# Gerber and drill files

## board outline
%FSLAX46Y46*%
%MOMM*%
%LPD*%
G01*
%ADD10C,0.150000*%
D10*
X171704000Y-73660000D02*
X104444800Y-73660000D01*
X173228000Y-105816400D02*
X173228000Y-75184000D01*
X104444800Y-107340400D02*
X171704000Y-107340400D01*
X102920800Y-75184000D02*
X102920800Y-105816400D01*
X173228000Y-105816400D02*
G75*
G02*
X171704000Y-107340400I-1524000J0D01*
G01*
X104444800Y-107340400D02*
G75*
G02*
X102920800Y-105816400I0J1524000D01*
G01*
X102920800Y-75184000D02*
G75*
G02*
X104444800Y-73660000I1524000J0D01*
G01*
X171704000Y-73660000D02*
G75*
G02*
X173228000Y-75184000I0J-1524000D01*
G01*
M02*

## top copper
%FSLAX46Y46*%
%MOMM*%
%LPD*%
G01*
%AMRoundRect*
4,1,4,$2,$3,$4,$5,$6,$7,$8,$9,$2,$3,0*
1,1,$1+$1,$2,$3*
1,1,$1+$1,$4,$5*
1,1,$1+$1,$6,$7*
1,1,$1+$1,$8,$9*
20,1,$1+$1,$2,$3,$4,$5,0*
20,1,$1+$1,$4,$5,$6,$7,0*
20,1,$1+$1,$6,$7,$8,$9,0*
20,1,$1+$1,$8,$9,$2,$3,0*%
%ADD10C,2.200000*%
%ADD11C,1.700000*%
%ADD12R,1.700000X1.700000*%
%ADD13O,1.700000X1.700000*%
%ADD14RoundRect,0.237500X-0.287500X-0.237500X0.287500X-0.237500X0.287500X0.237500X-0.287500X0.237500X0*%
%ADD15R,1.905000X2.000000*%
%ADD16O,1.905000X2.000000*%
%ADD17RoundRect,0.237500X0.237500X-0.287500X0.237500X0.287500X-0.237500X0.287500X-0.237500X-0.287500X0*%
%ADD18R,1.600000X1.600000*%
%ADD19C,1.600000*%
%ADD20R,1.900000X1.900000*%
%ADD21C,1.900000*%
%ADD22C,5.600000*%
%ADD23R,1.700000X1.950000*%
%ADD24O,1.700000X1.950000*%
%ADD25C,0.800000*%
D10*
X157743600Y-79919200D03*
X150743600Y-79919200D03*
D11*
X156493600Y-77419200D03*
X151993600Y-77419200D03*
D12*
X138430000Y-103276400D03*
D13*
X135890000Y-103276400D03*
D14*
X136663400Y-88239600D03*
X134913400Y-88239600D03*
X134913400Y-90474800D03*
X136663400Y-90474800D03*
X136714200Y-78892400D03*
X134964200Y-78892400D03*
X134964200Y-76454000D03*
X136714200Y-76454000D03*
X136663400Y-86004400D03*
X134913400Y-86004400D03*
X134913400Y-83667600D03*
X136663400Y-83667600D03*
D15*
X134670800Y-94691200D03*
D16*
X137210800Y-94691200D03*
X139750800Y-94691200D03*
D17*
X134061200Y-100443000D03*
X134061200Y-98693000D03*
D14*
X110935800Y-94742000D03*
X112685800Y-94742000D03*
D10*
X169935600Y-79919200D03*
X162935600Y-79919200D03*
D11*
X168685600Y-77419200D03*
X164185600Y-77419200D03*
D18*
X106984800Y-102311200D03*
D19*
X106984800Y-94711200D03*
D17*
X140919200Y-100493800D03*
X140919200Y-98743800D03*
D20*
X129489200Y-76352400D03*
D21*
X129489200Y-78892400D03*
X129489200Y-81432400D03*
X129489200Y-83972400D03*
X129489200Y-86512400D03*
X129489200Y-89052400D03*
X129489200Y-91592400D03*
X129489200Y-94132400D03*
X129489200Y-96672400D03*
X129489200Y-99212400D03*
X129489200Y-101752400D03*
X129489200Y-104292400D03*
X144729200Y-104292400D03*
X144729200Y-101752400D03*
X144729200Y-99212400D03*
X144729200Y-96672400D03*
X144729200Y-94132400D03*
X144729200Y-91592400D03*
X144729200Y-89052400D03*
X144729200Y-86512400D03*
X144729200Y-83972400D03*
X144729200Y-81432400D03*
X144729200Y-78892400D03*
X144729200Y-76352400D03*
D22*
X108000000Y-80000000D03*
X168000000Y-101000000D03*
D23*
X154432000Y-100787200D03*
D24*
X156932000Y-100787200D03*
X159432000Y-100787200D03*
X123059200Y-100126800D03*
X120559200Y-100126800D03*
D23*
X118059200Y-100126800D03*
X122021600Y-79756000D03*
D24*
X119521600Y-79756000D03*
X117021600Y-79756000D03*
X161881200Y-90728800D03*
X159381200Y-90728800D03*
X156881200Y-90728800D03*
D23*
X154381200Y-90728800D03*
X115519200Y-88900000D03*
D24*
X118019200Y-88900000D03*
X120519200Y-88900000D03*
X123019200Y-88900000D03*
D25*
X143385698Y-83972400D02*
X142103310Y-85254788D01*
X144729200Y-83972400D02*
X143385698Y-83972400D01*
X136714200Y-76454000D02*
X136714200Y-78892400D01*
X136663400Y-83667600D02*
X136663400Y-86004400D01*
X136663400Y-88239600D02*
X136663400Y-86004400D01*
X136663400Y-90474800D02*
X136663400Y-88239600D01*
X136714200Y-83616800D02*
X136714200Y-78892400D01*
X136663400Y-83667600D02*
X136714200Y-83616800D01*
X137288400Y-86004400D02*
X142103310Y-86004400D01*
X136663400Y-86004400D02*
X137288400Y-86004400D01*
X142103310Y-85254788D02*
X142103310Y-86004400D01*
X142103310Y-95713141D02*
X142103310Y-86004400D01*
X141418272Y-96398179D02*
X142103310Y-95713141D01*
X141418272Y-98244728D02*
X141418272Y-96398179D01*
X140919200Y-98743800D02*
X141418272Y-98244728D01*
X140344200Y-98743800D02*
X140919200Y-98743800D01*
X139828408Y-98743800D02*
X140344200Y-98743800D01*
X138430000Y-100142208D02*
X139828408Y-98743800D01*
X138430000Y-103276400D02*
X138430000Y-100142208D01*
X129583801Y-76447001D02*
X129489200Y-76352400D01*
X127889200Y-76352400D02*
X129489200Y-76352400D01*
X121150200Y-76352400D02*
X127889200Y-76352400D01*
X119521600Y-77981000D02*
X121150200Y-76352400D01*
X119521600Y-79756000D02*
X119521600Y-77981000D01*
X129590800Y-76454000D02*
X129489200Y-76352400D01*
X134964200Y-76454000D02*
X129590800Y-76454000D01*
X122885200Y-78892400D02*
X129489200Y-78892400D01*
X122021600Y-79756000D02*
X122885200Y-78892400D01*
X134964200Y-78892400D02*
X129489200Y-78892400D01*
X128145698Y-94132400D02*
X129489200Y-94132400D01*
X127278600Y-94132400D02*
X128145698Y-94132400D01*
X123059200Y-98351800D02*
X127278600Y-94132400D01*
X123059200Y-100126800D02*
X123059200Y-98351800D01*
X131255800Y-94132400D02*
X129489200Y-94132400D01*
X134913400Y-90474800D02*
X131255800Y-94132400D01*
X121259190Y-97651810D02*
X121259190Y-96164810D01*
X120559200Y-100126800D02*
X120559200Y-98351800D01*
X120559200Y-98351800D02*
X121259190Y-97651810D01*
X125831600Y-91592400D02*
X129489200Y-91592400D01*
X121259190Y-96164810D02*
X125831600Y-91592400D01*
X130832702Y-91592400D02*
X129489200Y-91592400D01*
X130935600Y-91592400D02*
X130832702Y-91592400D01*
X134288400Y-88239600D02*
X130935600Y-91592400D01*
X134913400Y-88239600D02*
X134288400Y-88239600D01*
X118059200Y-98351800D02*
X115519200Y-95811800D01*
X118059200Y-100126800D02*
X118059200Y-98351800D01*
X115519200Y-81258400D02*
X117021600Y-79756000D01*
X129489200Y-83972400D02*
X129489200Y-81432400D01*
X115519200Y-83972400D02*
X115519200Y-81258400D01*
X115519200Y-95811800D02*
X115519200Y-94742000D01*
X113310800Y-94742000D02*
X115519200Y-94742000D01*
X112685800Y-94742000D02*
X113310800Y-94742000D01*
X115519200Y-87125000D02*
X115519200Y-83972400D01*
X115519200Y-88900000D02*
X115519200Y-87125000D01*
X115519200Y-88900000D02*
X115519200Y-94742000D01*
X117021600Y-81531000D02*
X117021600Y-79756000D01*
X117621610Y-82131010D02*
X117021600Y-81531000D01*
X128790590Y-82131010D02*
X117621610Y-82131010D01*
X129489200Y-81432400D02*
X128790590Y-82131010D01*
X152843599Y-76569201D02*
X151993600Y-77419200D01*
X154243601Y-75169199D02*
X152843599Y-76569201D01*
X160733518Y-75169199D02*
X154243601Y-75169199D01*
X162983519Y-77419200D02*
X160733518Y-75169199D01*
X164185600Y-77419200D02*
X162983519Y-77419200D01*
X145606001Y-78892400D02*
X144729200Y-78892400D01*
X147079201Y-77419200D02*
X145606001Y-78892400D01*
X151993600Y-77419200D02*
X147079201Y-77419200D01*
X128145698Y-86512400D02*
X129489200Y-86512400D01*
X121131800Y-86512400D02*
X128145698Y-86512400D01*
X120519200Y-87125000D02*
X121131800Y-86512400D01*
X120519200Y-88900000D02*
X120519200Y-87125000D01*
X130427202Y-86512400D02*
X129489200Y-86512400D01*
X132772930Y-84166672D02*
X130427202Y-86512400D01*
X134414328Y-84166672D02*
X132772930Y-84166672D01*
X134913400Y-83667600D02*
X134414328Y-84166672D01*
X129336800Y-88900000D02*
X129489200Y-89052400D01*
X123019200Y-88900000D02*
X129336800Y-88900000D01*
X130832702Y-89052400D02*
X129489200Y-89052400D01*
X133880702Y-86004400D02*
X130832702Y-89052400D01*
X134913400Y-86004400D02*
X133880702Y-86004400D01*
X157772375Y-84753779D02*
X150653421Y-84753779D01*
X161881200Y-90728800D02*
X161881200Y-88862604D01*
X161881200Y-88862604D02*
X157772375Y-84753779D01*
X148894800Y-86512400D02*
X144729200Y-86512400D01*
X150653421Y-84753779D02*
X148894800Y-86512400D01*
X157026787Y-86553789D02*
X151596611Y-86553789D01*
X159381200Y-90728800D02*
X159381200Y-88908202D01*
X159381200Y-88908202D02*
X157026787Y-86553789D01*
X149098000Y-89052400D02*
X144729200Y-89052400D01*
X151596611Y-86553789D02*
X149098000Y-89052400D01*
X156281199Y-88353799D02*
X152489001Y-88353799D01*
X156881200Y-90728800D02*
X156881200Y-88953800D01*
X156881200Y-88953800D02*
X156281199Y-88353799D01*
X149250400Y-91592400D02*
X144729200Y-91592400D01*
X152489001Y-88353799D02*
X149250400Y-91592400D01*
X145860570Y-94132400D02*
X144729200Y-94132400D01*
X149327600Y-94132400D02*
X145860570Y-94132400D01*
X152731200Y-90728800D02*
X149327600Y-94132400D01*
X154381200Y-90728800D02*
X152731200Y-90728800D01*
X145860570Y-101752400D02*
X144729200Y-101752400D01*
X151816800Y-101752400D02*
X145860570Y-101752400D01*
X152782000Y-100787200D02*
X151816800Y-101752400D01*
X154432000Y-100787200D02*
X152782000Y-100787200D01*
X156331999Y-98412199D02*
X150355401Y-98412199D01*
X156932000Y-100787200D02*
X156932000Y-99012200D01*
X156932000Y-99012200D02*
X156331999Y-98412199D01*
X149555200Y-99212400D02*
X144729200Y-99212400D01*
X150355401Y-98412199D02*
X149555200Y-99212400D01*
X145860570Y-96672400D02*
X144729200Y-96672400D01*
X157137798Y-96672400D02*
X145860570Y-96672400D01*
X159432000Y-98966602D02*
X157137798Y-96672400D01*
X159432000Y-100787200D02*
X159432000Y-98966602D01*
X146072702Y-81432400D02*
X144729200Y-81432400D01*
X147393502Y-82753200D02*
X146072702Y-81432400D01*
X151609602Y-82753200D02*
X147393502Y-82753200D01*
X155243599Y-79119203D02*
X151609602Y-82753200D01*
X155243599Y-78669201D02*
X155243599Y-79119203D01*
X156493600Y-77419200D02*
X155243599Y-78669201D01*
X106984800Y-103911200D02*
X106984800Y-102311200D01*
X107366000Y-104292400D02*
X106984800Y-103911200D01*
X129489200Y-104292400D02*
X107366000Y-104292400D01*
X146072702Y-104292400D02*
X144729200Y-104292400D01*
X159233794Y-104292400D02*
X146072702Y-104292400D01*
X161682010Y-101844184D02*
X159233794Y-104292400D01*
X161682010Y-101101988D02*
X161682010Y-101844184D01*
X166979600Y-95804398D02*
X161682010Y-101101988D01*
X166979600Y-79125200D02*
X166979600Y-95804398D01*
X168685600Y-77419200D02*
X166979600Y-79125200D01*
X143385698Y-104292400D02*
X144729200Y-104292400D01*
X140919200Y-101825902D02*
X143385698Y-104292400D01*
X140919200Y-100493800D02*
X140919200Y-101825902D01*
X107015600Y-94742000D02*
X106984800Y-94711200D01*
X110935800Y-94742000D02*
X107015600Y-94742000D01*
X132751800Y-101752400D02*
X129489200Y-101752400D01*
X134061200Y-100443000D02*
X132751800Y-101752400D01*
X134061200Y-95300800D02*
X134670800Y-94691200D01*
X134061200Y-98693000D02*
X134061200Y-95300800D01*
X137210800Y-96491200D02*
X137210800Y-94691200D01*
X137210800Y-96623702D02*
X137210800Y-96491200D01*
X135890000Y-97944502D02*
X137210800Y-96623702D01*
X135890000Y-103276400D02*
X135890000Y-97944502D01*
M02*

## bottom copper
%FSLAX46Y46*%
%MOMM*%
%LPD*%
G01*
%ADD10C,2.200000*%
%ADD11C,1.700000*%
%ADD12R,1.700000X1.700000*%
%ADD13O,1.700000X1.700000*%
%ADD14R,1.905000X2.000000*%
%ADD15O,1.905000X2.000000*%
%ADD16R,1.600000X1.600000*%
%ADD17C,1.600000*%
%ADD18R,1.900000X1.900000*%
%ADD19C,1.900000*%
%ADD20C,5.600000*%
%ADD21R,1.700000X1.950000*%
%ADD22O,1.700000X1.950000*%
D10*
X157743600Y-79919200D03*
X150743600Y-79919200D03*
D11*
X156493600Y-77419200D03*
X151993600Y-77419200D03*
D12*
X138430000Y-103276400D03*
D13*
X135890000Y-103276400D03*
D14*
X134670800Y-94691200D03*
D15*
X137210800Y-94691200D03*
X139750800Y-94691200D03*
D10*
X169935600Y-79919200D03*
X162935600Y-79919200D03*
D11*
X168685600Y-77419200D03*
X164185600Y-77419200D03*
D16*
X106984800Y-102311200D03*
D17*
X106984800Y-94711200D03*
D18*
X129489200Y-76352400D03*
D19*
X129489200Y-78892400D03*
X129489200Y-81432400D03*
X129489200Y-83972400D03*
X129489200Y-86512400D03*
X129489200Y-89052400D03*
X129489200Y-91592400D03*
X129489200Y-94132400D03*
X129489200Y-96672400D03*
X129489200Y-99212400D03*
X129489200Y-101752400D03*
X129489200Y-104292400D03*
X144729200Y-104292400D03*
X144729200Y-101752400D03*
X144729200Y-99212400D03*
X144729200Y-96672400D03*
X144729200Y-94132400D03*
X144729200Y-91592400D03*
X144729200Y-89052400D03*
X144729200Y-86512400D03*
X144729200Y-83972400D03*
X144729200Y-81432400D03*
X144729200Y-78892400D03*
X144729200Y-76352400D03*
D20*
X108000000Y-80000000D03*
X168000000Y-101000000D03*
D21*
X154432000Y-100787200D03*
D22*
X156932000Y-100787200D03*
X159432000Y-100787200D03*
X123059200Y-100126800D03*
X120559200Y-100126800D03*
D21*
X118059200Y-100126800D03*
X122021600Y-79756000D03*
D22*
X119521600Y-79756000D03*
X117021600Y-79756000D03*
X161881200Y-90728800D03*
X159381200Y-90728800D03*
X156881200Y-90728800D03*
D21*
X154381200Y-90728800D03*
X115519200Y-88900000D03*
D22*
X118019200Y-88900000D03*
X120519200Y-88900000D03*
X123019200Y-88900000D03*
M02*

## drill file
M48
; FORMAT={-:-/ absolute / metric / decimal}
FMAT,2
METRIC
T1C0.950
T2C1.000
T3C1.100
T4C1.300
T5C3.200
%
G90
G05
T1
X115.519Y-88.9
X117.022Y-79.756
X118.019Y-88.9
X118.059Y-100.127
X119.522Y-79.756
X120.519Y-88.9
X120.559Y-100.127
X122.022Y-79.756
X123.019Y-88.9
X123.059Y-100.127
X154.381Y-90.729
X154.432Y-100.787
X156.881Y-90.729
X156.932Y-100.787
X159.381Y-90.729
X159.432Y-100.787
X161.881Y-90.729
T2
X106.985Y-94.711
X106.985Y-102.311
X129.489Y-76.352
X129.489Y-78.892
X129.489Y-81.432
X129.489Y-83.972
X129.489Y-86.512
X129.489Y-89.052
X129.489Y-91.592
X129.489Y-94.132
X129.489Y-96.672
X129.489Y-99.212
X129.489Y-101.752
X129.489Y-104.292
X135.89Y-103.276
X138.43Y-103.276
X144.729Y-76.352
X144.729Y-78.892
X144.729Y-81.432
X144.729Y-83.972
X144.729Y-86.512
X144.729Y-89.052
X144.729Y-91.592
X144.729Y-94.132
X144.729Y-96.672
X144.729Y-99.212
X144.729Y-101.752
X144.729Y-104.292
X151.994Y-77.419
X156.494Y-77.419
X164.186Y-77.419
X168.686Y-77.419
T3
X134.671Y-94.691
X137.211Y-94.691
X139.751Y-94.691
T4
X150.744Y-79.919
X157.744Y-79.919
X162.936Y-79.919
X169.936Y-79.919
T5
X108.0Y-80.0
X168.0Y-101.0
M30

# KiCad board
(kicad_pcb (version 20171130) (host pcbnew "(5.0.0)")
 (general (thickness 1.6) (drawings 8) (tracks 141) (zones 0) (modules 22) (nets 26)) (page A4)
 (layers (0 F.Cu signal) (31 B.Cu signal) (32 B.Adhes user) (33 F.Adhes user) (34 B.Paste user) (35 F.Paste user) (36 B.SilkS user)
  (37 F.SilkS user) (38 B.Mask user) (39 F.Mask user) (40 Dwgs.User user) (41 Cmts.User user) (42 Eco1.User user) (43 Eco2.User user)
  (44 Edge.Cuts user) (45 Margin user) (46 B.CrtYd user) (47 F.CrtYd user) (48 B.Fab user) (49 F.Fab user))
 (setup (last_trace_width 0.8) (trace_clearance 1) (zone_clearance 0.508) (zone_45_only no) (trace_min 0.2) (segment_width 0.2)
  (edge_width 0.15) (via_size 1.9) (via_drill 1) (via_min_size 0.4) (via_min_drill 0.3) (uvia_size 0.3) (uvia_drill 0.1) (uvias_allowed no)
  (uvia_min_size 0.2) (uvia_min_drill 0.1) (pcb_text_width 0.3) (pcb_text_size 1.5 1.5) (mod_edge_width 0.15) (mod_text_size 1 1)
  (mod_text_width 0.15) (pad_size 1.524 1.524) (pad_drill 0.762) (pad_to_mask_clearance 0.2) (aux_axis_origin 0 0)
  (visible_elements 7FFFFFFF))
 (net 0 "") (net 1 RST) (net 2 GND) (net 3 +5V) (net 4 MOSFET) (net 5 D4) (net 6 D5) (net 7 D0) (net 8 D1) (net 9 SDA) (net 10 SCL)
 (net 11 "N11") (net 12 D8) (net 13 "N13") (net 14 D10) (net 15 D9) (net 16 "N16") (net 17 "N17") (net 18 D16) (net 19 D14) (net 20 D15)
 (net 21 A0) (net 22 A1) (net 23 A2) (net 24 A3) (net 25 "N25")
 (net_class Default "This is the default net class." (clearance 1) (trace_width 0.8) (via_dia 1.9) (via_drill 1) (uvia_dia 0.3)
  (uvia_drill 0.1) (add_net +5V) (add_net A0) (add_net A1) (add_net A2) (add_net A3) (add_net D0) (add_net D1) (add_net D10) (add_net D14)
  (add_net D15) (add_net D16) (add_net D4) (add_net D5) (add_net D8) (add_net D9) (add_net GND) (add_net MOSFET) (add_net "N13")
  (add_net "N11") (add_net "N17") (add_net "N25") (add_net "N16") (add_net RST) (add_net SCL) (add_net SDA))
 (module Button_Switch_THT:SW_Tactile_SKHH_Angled (layer F.Cu) (at 151.9936 77.4192)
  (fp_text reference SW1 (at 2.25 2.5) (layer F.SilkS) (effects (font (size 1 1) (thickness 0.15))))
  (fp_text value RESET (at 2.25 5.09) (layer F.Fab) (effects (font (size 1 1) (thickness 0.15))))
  (pad "" thru_hole circle (at 5.75 2.5 180) (size 2.2 2.2) (drill 1.3) (layers *.Cu *.Mask))
  (pad "" thru_hole circle (at -1.25 2.5 180) (size 2.2 2.2) (drill 1.3) (layers *.Cu *.Mask))
  (pad 2 thru_hole circle (at 4.5 0 180) (size 1.7 1.7) (drill 1) (layers *.Cu *.Mask) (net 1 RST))
  (pad 1 thru_hole circle (at 0 0 180) (size 1.7 1.7) (drill 1) (layers *.Cu *.Mask) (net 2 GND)))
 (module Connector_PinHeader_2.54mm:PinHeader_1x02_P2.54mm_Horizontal (layer F.Cu) (at 138.43 103.2764 270)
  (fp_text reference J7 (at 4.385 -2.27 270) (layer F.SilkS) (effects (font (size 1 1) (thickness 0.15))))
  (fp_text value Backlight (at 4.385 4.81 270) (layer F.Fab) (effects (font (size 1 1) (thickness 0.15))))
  (pad 1 thru_hole rect (at 0 0 270) (size 1.7 1.7) (drill 1) (layers *.Cu *.Mask) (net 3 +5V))
  (pad 2 thru_hole oval (at 0 2.54 270) (size 1.7 1.7) (drill 1) (layers *.Cu *.Mask) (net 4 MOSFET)))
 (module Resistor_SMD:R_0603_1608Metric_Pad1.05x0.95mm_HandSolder (layer F.Cu) (at 135.7884 88.2396)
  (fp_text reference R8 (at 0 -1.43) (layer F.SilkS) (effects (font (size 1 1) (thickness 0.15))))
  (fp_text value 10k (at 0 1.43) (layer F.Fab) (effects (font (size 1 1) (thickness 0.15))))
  (pad 2 smd roundrect (at 0.875 0) (size 1.05 0.95) (layers F.Cu F.Paste F.Mask) (roundrect_rratio 0.25) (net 3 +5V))
  (pad 1 smd roundrect (at -0.875 0) (size 1.05 0.95) (layers F.Cu F.Paste F.Mask) (roundrect_rratio 0.25) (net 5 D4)))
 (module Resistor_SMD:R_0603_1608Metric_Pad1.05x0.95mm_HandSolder (layer F.Cu) (at 135.7884 90.4748)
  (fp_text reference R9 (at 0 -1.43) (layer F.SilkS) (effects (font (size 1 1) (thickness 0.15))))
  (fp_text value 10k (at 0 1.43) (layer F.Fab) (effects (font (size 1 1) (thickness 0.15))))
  (pad 1 smd roundrect (at -0.875 0) (size 1.05 0.95) (layers F.Cu F.Paste F.Mask) (roundrect_rratio 0.25) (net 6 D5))
  (pad 2 smd roundrect (at 0.875 0) (size 1.05 0.95) (layers F.Cu F.Paste F.Mask) (roundrect_rratio 0.25) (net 3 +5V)))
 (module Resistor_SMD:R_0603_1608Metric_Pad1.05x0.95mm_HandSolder (layer F.Cu) (at 135.8392 78.8924)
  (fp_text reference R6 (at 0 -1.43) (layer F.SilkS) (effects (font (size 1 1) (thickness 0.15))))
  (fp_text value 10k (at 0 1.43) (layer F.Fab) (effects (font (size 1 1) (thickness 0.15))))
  (pad 2 smd roundrect (at 0.875 0) (size 1.05 0.95) (layers F.Cu F.Paste F.Mask) (roundrect_rratio 0.25) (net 3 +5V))
  (pad 1 smd roundrect (at -0.875 0) (size 1.05 0.95) (layers F.Cu F.Paste F.Mask) (roundrect_rratio 0.25) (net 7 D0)))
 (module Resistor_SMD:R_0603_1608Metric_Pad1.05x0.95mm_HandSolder (layer F.Cu) (at 135.8392 76.454)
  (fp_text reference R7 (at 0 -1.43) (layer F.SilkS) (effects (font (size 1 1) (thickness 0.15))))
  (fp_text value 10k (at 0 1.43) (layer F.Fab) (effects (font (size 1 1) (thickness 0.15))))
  (pad 1 smd roundrect (at -0.875 0) (size 1.05 0.95) (layers F.Cu F.Paste F.Mask) (roundrect_rratio 0.25) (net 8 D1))
  (pad 2 smd roundrect (at 0.875 0) (size 1.05 0.95) (layers F.Cu F.Paste F.Mask) (roundrect_rratio 0.25) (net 3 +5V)))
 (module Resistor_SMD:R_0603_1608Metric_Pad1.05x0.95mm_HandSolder (layer F.Cu) (at 135.7884 86.0044)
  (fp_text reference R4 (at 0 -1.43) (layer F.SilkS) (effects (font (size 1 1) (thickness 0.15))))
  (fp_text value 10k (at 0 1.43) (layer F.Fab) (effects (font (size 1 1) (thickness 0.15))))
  (pad 2 smd roundrect (at 0.875 0) (size 1.05 0.95) (layers F.Cu F.Paste F.Mask) (roundrect_rratio 0.25) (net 3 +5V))
  (pad 1 smd roundrect (at -0.875 0) (size 1.05 0.95) (layers F.Cu F.Paste F.Mask) (roundrect_rratio 0.25) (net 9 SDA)))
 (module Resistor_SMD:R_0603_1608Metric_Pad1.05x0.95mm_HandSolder (layer F.Cu) (at 135.7884 83.6676)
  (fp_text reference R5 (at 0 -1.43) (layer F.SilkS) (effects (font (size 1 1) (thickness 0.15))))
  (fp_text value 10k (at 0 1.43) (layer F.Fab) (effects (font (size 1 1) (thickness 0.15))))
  (pad 1 smd roundrect (at -0.875 0) (size 1.05 0.95) (layers F.Cu F.Paste F.Mask) (roundrect_rratio 0.25) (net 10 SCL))
  (pad 2 smd roundrect (at 0.875 0) (size 1.05 0.95) (layers F.Cu F.Paste F.Mask) (roundrect_rratio 0.25) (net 3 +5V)))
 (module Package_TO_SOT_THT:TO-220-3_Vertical (layer F.Cu) (at 134.6708 94.6912)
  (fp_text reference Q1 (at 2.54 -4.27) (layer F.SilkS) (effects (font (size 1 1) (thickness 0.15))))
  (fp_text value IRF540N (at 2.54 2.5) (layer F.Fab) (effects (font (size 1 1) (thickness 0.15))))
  (pad 1 thru_hole rect (at 0 0) (size 1.905 2) (drill 1.1) (layers *.Cu *.Mask) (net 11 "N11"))
  (pad 2 thru_hole oval (at 2.54 0) (size 1.905 2) (drill 1.1) (layers *.Cu *.Mask) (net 4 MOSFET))
  (pad 3 thru_hole oval (at 5.08 0) (size 1.905 2) (drill 1.1) (layers *.Cu *.Mask) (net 2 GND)))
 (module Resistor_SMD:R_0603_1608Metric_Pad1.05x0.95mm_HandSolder (layer F.Cu) (at 134.0612 99.568 90)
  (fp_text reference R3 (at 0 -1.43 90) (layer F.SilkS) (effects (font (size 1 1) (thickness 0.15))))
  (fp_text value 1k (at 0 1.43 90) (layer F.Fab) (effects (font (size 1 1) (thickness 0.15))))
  (pad 1 smd roundrect (at -0.875 0 90) (size 1.05 0.95) (layers F.Cu F.Paste F.Mask) (roundrect_rratio 0.25) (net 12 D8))
  (pad 2 smd roundrect (at 0.875 0 90) (size 1.05 0.95) (layers F.Cu F.Paste F.Mask) (roundrect_rratio 0.25) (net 11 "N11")))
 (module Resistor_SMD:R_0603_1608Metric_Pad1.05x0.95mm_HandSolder (layer F.Cu) (at 111.8108 94.742)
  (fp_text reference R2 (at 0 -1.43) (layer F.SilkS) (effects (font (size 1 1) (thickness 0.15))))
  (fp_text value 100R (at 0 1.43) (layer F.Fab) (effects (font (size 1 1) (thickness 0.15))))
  (pad 1 smd roundrect (at -0.875 0) (size 1.05 0.95) (layers F.Cu F.Paste F.Mask) (roundrect_rratio 0.25) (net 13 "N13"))
  (pad 2 smd roundrect (at 0.875 0) (size 1.05 0.95) (layers F.Cu F.Paste F.Mask) (roundrect_rratio 0.25) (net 2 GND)))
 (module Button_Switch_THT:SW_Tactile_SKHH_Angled (layer F.Cu) (at 164.1856 77.4192)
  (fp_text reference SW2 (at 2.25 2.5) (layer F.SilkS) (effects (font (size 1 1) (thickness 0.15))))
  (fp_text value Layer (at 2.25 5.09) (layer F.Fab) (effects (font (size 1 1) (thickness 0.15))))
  (pad "" thru_hole circle (at 5.75 2.5 180) (size 2.2 2.2) (drill 1.3) (layers *.Cu *.Mask))
  (pad "" thru_hole circle (at -1.25 2.5 180) (size 2.2 2.2) (drill 1.3) (layers *.Cu *.Mask))
  (pad 2 thru_hole circle (at 4.5 0 180) (size 1.7 1.7) (drill 1) (layers *.Cu *.Mask) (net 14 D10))
  (pad 1 thru_hole circle (at 0 0 180) (size 1.7 1.7) (drill 1) (layers *.Cu *.Mask) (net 2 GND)))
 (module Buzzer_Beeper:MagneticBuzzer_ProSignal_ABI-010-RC (layer F.Cu) (at 106.9848 102.3112 90)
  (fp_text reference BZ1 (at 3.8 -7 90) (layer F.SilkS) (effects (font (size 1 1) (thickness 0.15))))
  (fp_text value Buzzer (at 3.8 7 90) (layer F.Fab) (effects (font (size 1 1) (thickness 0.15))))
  (pad 1 thru_hole rect (at 0 0 90) (size 1.6 1.6) (drill 1) (layers *.Cu *.Mask) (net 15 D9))
  (pad 2 thru_hole circle (at 7.6 0 90) (size 1.6 1.6) (drill 1) (layers *.Cu *.Mask) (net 13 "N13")))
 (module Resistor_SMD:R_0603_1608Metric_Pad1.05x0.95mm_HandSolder (layer F.Cu) (at 140.9192 99.6188 90)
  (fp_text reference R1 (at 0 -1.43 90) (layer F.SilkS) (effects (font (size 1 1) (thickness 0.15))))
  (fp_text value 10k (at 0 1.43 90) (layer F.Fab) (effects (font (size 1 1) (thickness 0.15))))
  (pad 1 smd roundrect (at -0.875 0 90) (size 1.05 0.95) (layers F.Cu F.Paste F.Mask) (roundrect_rratio 0.25) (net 14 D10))
  (pad 2 smd roundrect (at 0.875 0 90) (size 1.05 0.95) (layers F.Cu F.Paste F.Mask) (roundrect_rratio 0.25) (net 3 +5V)))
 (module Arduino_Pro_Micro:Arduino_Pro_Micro (layer F.Cu) (at 137.1092 90.3224 270)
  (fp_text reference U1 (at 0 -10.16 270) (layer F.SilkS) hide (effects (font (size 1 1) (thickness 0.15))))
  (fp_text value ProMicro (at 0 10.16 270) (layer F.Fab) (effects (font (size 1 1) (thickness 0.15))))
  (pad 1 thru_hole rect (at -13.97 7.62 270) (size 1.9 1.9) (drill 1) (layers *.Cu *.Mask F.SilkS) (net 8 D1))
  (pad 2 thru_hole circle (at -11.43 7.62 270) (size 1.9 1.9) (drill 1) (layers *.Cu *.Mask F.SilkS) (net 7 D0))
  (pad 3 thru_hole circle (at -8.89 7.62 270) (size 1.9 1.9) (drill 1) (layers *.Cu *.Mask F.SilkS) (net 2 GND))
  (pad 4 thru_hole circle (at -6.35 7.62 270) (size 1.9 1.9) (drill 1) (layers *.Cu *.Mask F.SilkS) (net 2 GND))
  (pad 5 thru_hole circle (at -3.81 7.62 270) (size 1.9 1.9) (drill 1) (layers *.Cu *.Mask F.SilkS) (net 10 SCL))
  (pad 6 thru_hole circle (at -1.27 7.62 270) (size 1.9 1.9) (drill 1) (layers *.Cu *.Mask F.SilkS) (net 9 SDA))
  (pad 7 thru_hole circle (at 1.27 7.62 270) (size 1.9 1.9) (drill 1) (layers *.Cu *.Mask F.SilkS) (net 5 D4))
  (pad 8 thru_hole circle (at 3.81 7.62 270) (size 1.9 1.9) (drill 1) (layers *.Cu *.Mask F.SilkS) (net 6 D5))
  (pad 9 thru_hole circle (at 6.35 7.62 270) (size 1.9 1.9) (drill 1) (layers *.Cu *.Mask F.SilkS) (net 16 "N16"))
  (pad 10 thru_hole circle (at 8.89 7.62 270) (size 1.9 1.9) (drill 1) (layers *.Cu *.Mask F.SilkS) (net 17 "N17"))
  (pad 11 thru_hole circle (at 11.43 7.62 270) (size 1.9 1.9) (drill 1) (layers *.Cu *.Mask F.SilkS) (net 12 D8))
  (pad 12 thru_hole circle (at 13.97 7.62 270) (size 1.9 1.9) (drill 1) (layers *.Cu *.Mask F.SilkS) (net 15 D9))
  (pad 13 thru_hole circle (at 13.97 -7.62 270) (size 1.9 1.9) (drill 1) (layers *.Cu *.Mask F.SilkS) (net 14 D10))
  (pad 14 thru_hole circle (at 11.43 -7.62 270) (size 1.9 1.9) (drill 1) (layers *.Cu *.Mask F.SilkS) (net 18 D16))
  (pad 15 thru_hole circle (at 8.89 -7.62 270) (size 1.9 1.9) (drill 1) (layers *.Cu *.Mask F.SilkS) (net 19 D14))
  (pad 16 thru_hole circle (at 6.35 -7.62 270) (size 1.9 1.9) (drill 1) (layers *.Cu *.Mask F.SilkS) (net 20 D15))
  (pad 17 thru_hole circle (at 3.81 -7.62 270) (size 1.9 1.9) (drill 1) (layers *.Cu *.Mask F.SilkS) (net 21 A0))
  (pad 18 thru_hole circle (at 1.27 -7.62 270) (size 1.9 1.9) (drill 1) (layers *.Cu *.Mask F.SilkS) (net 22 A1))
  (pad 19 thru_hole circle (at -1.27 -7.62 270) (size 1.9 1.9) (drill 1) (layers *.Cu *.Mask F.SilkS) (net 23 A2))
  (pad 20 thru_hole circle (at -3.81 -7.62 270) (size 1.9 1.9) (drill 1) (layers *.Cu *.Mask F.SilkS) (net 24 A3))
  (pad 21 thru_hole circle (at -6.35 -7.62 270) (size 1.9 1.9) (drill 1) (layers *.Cu *.Mask F.SilkS) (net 3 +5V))
  (pad 22 thru_hole circle (at -8.89 -7.62 270) (size 1.9 1.9) (drill 1) (layers *.Cu *.Mask F.SilkS) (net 1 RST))
  (pad 23 thru_hole circle (at -11.43 -7.62 270) (size 1.9 1.9) (drill 1) (layers *.Cu *.Mask F.SilkS) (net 2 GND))
  (pad 24 thru_hole circle (at -13.97 -7.62 270) (size 1.9 1.9) (drill 1) (layers *.Cu *.Mask F.SilkS) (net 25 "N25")))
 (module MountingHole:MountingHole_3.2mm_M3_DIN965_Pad (layer F.Cu) (at 108 80)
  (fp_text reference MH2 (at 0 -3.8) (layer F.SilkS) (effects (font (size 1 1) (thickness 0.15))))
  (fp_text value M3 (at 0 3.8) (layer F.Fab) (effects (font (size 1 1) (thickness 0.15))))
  (pad 1 thru_hole circle (at 0 0) (size 5.6 5.6) (drill 3.2) (layers *.Cu *.Mask)))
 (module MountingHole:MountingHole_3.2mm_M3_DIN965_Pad (layer F.Cu) (at 168 101)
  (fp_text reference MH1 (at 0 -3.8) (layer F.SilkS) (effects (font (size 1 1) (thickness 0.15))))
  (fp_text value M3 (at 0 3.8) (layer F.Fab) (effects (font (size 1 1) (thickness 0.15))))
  (pad 1 thru_hole circle (at 0 0) (size 5.6 5.6) (drill 3.2) (layers *.Cu *.Mask)))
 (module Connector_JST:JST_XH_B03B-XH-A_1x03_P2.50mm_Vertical (layer F.Cu) (at 154.432 100.7872)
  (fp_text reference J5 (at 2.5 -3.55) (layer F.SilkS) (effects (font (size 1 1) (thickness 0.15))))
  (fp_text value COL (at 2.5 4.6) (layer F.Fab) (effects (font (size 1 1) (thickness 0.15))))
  (pad 1 thru_hole rect (at 0 0) (size 1.7 1.95) (drill 0.95) (layers *.Cu *.Mask) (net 18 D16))
  (pad 2 thru_hole oval (at 2.5 0) (size 1.7 1.95) (drill 0.95) (layers *.Cu *.Mask) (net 19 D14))
  (pad 3 thru_hole oval (at 5 0) (size 1.7 1.95) (drill 0.95) (layers *.Cu *.Mask) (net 20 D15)))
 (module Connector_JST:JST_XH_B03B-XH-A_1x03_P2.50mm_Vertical (layer F.Cu) (at 118.0592 100.1268)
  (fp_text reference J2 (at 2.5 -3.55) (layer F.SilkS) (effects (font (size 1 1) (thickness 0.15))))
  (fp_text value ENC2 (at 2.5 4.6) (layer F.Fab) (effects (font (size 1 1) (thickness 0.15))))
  (pad 3 thru_hole oval (at 5 0) (size 1.7 1.95) (drill 0.95) (layers *.Cu *.Mask) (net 6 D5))
  (pad 2 thru_hole oval (at 2.5 0) (size 1.7 1.95) (drill 0.95) (layers *.Cu *.Mask) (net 5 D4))
  (pad 1 thru_hole rect (at 0 0) (size 1.7 1.95) (drill 0.95) (layers *.Cu *.Mask) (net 2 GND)))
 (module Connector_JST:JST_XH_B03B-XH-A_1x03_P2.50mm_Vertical (layer F.Cu) (at 122.0216 79.756 180)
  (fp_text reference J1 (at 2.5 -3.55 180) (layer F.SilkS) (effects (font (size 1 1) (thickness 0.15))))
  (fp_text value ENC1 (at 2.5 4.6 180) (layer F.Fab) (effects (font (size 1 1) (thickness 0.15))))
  (pad 1 thru_hole rect (at 0 0 180) (size 1.7 1.95) (drill 0.95) (layers *.Cu *.Mask) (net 7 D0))
  (pad 2 thru_hole oval (at 2.5 0 180) (size 1.7 1.95) (drill 0.95) (layers *.Cu *.Mask) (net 8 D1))
  (pad 3 thru_hole oval (at 5 0 180) (size 1.7 1.95) (drill 0.95) (layers *.Cu *.Mask) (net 2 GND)))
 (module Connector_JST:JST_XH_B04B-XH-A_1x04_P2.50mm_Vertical (layer F.Cu) (at 154.3812 90.7288)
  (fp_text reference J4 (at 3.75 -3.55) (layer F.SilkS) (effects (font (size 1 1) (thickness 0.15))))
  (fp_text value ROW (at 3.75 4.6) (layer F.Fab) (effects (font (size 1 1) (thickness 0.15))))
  (pad 4 thru_hole oval (at 7.5 0) (size 1.7 1.95) (drill 0.95) (layers *.Cu *.Mask) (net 24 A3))
  (pad 3 thru_hole oval (at 5 0) (size 1.7 1.95) (drill 0.95) (layers *.Cu *.Mask) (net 23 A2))
  (pad 2 thru_hole oval (at 2.5 0) (size 1.7 1.95) (drill 0.95) (layers *.Cu *.Mask) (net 22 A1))
  (pad 1 thru_hole rect (at 0 0) (size 1.7 1.95) (drill 0.95) (layers *.Cu *.Mask) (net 21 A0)))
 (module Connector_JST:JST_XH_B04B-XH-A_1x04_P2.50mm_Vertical (layer F.Cu) (at 115.5192 88.9)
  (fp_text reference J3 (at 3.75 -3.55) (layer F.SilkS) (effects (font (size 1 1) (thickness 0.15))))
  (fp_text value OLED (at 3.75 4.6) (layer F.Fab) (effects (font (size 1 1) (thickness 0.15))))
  (pad 1 thru_hole rect (at 0 0) (size 1.7 1.95) (drill 0.95) (layers *.Cu *.Mask) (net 2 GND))
  (pad 2 thru_hole oval (at 2.5 0) (size 1.7 1.95) (drill 0.95) (layers *.Cu *.Mask) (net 3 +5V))
  (pad 3 thru_hole oval (at 5 0) (size 1.7 1.95) (drill 0.95) (layers *.Cu *.Mask) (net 10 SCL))
  (pad 4 thru_hole oval (at 7.5 0) (size 1.7 1.95) (drill 0.95) (layers *.Cu *.Mask) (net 9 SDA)))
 (gr_line (start 171.704 73.66) (end 104.4448 73.66) (layer Edge.Cuts) (width 0.15))
 (gr_line (start 173.228 105.8164) (end 173.228 75.184) (layer Edge.Cuts) (width 0.15))
 (gr_line (start 104.4448 107.3404) (end 171.704 107.3404) (layer Edge.Cuts) (width 0.15))
 (gr_line (start 102.9208 75.184) (end 102.9208 105.8164) (layer Edge.Cuts) (width 0.15))
 (gr_arc (start 171.704 105.8164) (end 171.704 107.3404) (angle -90) (layer Edge.Cuts) (width 0.15))
 (gr_arc (start 104.4448 105.8164) (end 102.9208 105.8164) (angle -90) (layer Edge.Cuts) (width 0.15))
 (gr_arc (start 104.4448 75.184) (end 104.4448 73.66) (angle -90) (layer Edge.Cuts) (width 0.15))
 (gr_arc (start 171.704 75.184) (end 173.228 75.184) (angle -90) (layer Edge.Cuts) (width 0.15))
 (segment (start 143.385698 83.9724) (end 142.10331 85.254788) (width 0.8) (layer F.Cu) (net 3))
 (segment (start 144.7292 83.9724) (end 143.385698 83.9724) (width 0.8) (layer F.Cu) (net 3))
 (segment (start 136.7142 76.454) (end 136.7142 78.8924) (width 0.8) (layer F.Cu) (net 3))
 (segment (start 136.6634 83.6676) (end 136.6634 86.0044) (width 0.8) (layer F.Cu) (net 3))
 (segment (start 136.6634 88.2396) (end 136.6634 86.0044) (width 0.8) (layer F.Cu) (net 3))
 (segment (start 136.6634 90.4748) (end 136.6634 88.2396) (width 0.8) (layer F.Cu) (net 3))
 (segment (start 136.7142 83.6168) (end 136.7142 78.8924) (width 0.8) (layer F.Cu) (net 3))
 (segment (start 136.6634 83.6676) (end 136.7142 83.6168) (width 0.8) (layer F.Cu) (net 3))
 (segment (start 137.2884 86.0044) (end 142.10331 86.0044) (width 0.8) (layer F.Cu) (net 3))
 (segment (start 136.6634 86.0044) (end 137.2884 86.0044) (width 0.8) (layer F.Cu) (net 3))
 (segment (start 142.10331 85.254788) (end 142.10331 86.0044) (width 0.8) (layer F.Cu) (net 3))
 (segment (start 142.10331 95.713141) (end 142.10331 86.0044) (width 0.8) (layer F.Cu) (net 3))
 (segment (start 141.418272 96.398179) (end 142.10331 95.713141) (width 0.8) (layer F.Cu) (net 3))
 (segment (start 141.418272 98.244728) (end 141.418272 96.398179) (width 0.8) (layer F.Cu) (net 3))
 (segment (start 140.9192 98.7438) (end 141.418272 98.244728) (width 0.8) (layer F.Cu) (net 3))
 (segment (start 140.3442 98.7438) (end 140.9192 98.7438) (width 0.8) (layer F.Cu) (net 3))
 (segment (start 139.828408 98.7438) (end 140.3442 98.7438) (width 0.8) (layer F.Cu) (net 3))
 (segment (start 138.43 100.142208) (end 139.828408 98.7438) (width 0.8) (layer F.Cu) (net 3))
 (segment (start 138.43 103.2764) (end 138.43 100.142208) (width 0.8) (layer F.Cu) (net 3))
 (segment (start 129.583801 76.447001) (end 129.4892 76.3524) (width 0.8) (layer F.Cu) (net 8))
 (segment (start 127.8892 76.3524) (end 129.4892 76.3524) (width 0.8) (layer F.Cu) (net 8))
 (segment (start 121.1502 76.3524) (end 127.8892 76.3524) (width 0.8) (layer F.Cu) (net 8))
 (segment (start 119.5216 77.981) (end 121.1502 76.3524) (width 0.8) (layer F.Cu) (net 8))
 (segment (start 119.5216 79.756) (end 119.5216 77.981) (width 0.8) (layer F.Cu) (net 8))
 (segment (start 129.5908 76.454) (end 129.4892 76.3524) (width 0.8) (layer F.Cu) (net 8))
 (segment (start 134.9642 76.454) (end 129.5908 76.454) (width 0.8) (layer F.Cu) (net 8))
 (segment (start 122.8852 78.8924) (end 129.4892 78.8924) (width 0.8) (layer F.Cu) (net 7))
 (segment (start 122.0216 79.756) (end 122.8852 78.8924) (width 0.8) (layer F.Cu) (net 7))
 (segment (start 134.9642 78.8924) (end 129.4892 78.8924) (width 0.8) (layer F.Cu) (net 7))
 (segment (start 128.145698 94.1324) (end 129.4892 94.1324) (width 0.8) (layer F.Cu) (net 6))
 (segment (start 127.2786 94.1324) (end 128.145698 94.1324) (width 0.8) (layer F.Cu) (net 6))
 (segment (start 123.0592 98.3518) (end 127.2786 94.1324) (width 0.8) (layer F.Cu) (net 6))
 (segment (start 123.0592 100.1268) (end 123.0592 98.3518) (width 0.8) (layer F.Cu) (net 6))
 (segment (start 131.2558 94.1324) (end 129.4892 94.1324) (width 0.8) (layer F.Cu) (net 6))
 (segment (start 134.9134 90.4748) (end 131.2558 94.1324) (width 0.8) (layer F.Cu) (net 6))
 (segment (start 121.25919 97.65181) (end 121.25919 96.16481) (width 0.8) (layer F.Cu) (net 5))
 (segment (start 120.5592 100.1268) (end 120.5592 98.3518) (width 0.8) (layer F.Cu) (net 5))
 (segment (start 120.5592 98.3518) (end 121.25919 97.65181) (width 0.8) (layer F.Cu) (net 5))
 (segment (start 125.8316 91.5924) (end 129.4892 91.5924) (width 0.8) (layer F.Cu) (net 5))
 (segment (start 121.25919 96.16481) (end 125.8316 91.5924) (width 0.8) (layer F.Cu) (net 5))
 (segment (start 130.832702 91.5924) (end 129.4892 91.5924) (width 0.8) (layer F.Cu) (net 5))
 (segment (start 130.9356 91.5924) (end 130.832702 91.5924) (width 0.8) (layer F.Cu) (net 5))
 (segment (start 134.2884 88.2396) (end 130.9356 91.5924) (width 0.8) (layer F.Cu) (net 5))
 (segment (start 134.9134 88.2396) (end 134.2884 88.2396) (width 0.8) (layer F.Cu) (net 5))
 (segment (start 118.0592 98.3518) (end 115.5192 95.8118) (width 0.8) (layer F.Cu) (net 2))
 (segment (start 118.0592 100.1268) (end 118.0592 98.3518) (width 0.8) (layer F.Cu) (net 2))
 (segment (start 115.5192 81.2584) (end 117.0216 79.756) (width 0.8) (layer F.Cu) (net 2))
 (segment (start 129.4892 83.9724) (end 129.4892 81.4324) (width 0.8) (layer F.Cu) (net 2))
 (segment (start 115.5192 83.9724) (end 115.5192 81.2584) (width 0.8) (layer F.Cu) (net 2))
 (segment (start 115.5192 95.8118) (end 115.5192 94.742) (width 0.8) (layer F.Cu) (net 2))
 (segment (start 113.3108 94.742) (end 115.5192 94.742) (width 0.8) (layer F.Cu) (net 2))
 (segment (start 112.6858 94.742) (end 113.3108 94.742) (width 0.8) (layer F.Cu) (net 2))
 (segment (start 115.5192 87.125) (end 115.5192 83.9724) (width 0.8) (layer F.Cu) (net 2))
 (segment (start 115.5192 88.9) (end 115.5192 87.125) (width 0.8) (layer F.Cu) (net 2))
 (segment (start 115.5192 88.9) (end 115.5192 94.742) (width 0.8) (layer F.Cu) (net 2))
 (segment (start 117.0216 81.531) (end 117.0216 79.756) (width 0.8) (layer F.Cu) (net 2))
 (segment (start 117.62161 82.13101) (end 117.0216 81.531) (width 0.8) (layer F.Cu) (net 2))
 (segment (start 128.79059 82.13101) (end 117.62161 82.13101) (width 0.8) (layer F.Cu) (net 2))
 (segment (start 129.4892 81.4324) (end 128.79059 82.13101) (width 0.8) (layer F.Cu) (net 2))
 (segment (start 152.843599 76.569201) (end 151.9936 77.4192) (width 0.8) (layer F.Cu) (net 2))
 (segment (start 154.243601 75.169199) (end 152.843599 76.569201) (width 0.8) (layer F.Cu) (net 2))
 (segment (start 160.733518 75.169199) (end 154.243601 75.169199) (width 0.8) (layer F.Cu) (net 2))
 (segment (start 162.983519 77.4192) (end 160.733518 75.169199) (width 0.8) (layer F.Cu) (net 2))
 (segment (start 164.1856 77.4192) (end 162.983519 77.4192) (width 0.8) (layer F.Cu) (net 2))
 (segment (start 145.606001 78.8924) (end 144.7292 78.8924) (width 0.8) (layer F.Cu) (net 2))
 (segment (start 147.079201 77.4192) (end 145.606001 78.8924) (width 0.8) (layer F.Cu) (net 2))
 (segment (start 151.9936 77.4192) (end 147.079201 77.4192) (width 0.8) (layer F.Cu) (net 2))
 (segment (start 128.145698 86.5124) (end 129.4892 86.5124) (width 0.8) (layer F.Cu) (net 10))
 (segment (start 121.1318 86.5124) (end 128.145698 86.5124) (width 0.8) (layer F.Cu) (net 10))
 (segment (start 120.5192 87.125) (end 121.1318 86.5124) (width 0.8) (layer F.Cu) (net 10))
 (segment (start 120.5192 88.9) (end 120.5192 87.125) (width 0.8) (layer F.Cu) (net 10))
 (segment (start 130.427202 86.5124) (end 129.4892 86.5124) (width 0.8) (layer F.Cu) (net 10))
 (segment (start 132.77293 84.166672) (end 130.427202 86.5124) (width 0.8) (layer F.Cu) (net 10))
 (segment (start 134.414328 84.166672) (end 132.77293 84.166672) (width 0.8) (layer F.Cu) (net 10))
 (segment (start 134.9134 83.6676) (end 134.414328 84.166672) (width 0.8) (layer F.Cu) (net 10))
 (segment (start 129.3368 88.9) (end 129.4892 89.0524) (width 0.8) (layer F.Cu) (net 9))
 (segment (start 123.0192 88.9) (end 129.3368 88.9) (width 0.8) (layer F.Cu) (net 9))
 (segment (start 130.832702 89.0524) (end 129.4892 89.0524) (width 0.8) (layer F.Cu) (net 9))
 (segment (start 133.880702 86.0044) (end 130.832702 89.0524) (width 0.8) (layer F.Cu) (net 9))
 (segment (start 134.9134 86.0044) (end 133.880702 86.0044) (width 0.8) (layer F.Cu) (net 9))
 (segment (start 157.772375 84.753779) (end 150.653421 84.753779) (width 0.8) (layer F.Cu) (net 24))
 (segment (start 161.8812 90.7288) (end 161.8812 88.862604) (width 0.8) (layer F.Cu) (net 24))
 (segment (start 161.8812 88.862604) (end 157.772375 84.753779) (width 0.8) (layer F.Cu) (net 24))
 (segment (start 148.8948 86.5124) (end 144.7292 86.5124) (width 0.8) (layer F.Cu) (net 24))
 (segment (start 150.653421 84.753779) (end 148.8948 86.5124) (width 0.8) (layer F.Cu) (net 24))
 (segment (start 157.026787 86.553789) (end 151.596611 86.553789) (width 0.8) (layer F.Cu) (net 23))
 (segment (start 159.3812 90.7288) (end 159.3812 88.908202) (width 0.8) (layer F.Cu) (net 23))
 (segment (start 159.3812 88.908202) (end 157.026787 86.553789) (width 0.8) (layer F.Cu) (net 23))
 (segment (start 149.098 89.0524) (end 144.7292 89.0524) (width 0.8) (layer F.Cu) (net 23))
 (segment (start 151.596611 86.553789) (end 149.098 89.0524) (width 0.8) (layer F.Cu) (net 23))
 (segment (start 156.281199 88.353799) (end 152.489001 88.353799) (width 0.8) (layer F.Cu) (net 22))
 (segment (start 156.8812 90.7288) (end 156.8812 88.9538) (width 0.8) (layer F.Cu) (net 22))
 (segment (start 156.8812 88.9538) (end 156.281199 88.353799) (width 0.8) (layer F.Cu) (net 22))
 (segment (start 149.2504 91.5924) (end 144.7292 91.5924) (width 0.8) (layer F.Cu) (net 22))
 (segment (start 152.489001 88.353799) (end 149.2504 91.5924) (width 0.8) (layer F.Cu) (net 22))
 (segment (start 145.86057 94.1324) (end 144.7292 94.1324) (width 0.8) (layer F.Cu) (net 21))
 (segment (start 149.3276 94.1324) (end 145.86057 94.1324) (width 0.8) (layer F.Cu) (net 21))
 (segment (start 152.7312 90.7288) (end 149.3276 94.1324) (width 0.8) (layer F.Cu) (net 21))
 (segment (start 154.3812 90.7288) (end 152.7312 90.7288) (width 0.8) (layer F.Cu) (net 21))
 (segment (start 145.86057 101.7524) (end 144.7292 101.7524) (width 0.8) (layer F.Cu) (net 18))
 (segment (start 151.8168 101.7524) (end 145.86057 101.7524) (width 0.8) (layer F.Cu) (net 18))
 (segment (start 152.782 100.7872) (end 151.8168 101.7524) (width 0.8) (layer F.Cu) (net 18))
 (segment (start 154.432 100.7872) (end 152.782 100.7872) (width 0.8) (layer F.Cu) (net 18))
 (segment (start 156.331999 98.412199) (end 150.355401 98.412199) (width 0.8) (layer F.Cu) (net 19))
 (segment (start 156.932 100.7872) (end 156.932 99.0122) (width 0.8) (layer F.Cu) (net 19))
 (segment (start 156.932 99.0122) (end 156.331999 98.412199) (width 0.8) (layer F.Cu) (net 19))
 (segment (start 149.5552 99.2124) (end 144.7292 99.2124) (width 0.8) (layer F.Cu) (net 19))
 (segment (start 150.355401 98.412199) (end 149.5552 99.2124) (width 0.8) (layer F.Cu) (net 19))
 (segment (start 145.86057 96.6724) (end 144.7292 96.6724) (width 0.8) (layer F.Cu) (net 20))
 (segment (start 157.137798 96.6724) (end 145.86057 96.6724) (width 0.8) (layer F.Cu) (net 20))
 (segment (start 159.432 98.966602) (end 157.137798 96.6724) (width 0.8) (layer F.Cu) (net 20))
 (segment (start 159.432 100.7872) (end 159.432 98.966602) (width 0.8) (layer F.Cu) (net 20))
 (segment (start 146.072702 81.4324) (end 144.7292 81.4324) (width 0.8) (layer F.Cu) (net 1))
 (segment (start 147.393502 82.7532) (end 146.072702 81.4324) (width 0.8) (layer F.Cu) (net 1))
 (segment (start 151.609602 82.7532) (end 147.393502 82.7532) (width 0.8) (layer F.Cu) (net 1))
 (segment (start 155.243599 79.119203) (end 151.609602 82.7532) (width 0.8) (layer F.Cu) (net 1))
 (segment (start 155.243599 78.669201) (end 155.243599 79.119203) (width 0.8) (layer F.Cu) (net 1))
 (segment (start 156.4936 77.4192) (end 155.243599 78.669201) (width 0.8) (layer F.Cu) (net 1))
 (segment (start 106.9848 103.9112) (end 106.9848 102.3112) (width 0.8) (layer F.Cu) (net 15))
 (segment (start 107.366 104.2924) (end 106.9848 103.9112) (width 0.8) (layer F.Cu) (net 15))
 (segment (start 129.4892 104.2924) (end 107.366 104.2924) (width 0.8) (layer F.Cu) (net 15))
 (segment (start 146.072702 104.2924) (end 144.7292 104.2924) (width 0.8) (layer F.Cu) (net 14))
 (segment (start 159.233794 104.2924) (end 146.072702 104.2924) (width 0.8) (layer F.Cu) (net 14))
 (segment (start 161.68201 101.844184) (end 159.233794 104.2924) (width 0.8) (layer F.Cu) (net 14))
 (segment (start 161.68201 101.101988) (end 161.68201 101.844184) (width 0.8) (layer F.Cu) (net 14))
 (segment (start 166.9796 95.804398) (end 161.68201 101.101988) (width 0.8) (layer F.Cu) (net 14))
 (segment (start 166.9796 79.1252) (end 166.9796 95.804398) (width 0.8) (layer F.Cu) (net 14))
 (segment (start 168.6856 77.4192) (end 166.9796 79.1252) (width 0.8) (layer F.Cu) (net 14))
 (segment (start 143.385698 104.2924) (end 144.7292 104.2924) (width 0.8) (layer F.Cu) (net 14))
 (segment (start 140.9192 101.825902) (end 143.385698 104.2924) (width 0.8) (layer F.Cu) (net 14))
 (segment (start 140.9192 100.4938) (end 140.9192 101.825902) (width 0.8) (layer F.Cu) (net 14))
 (segment (start 107.0156 94.742) (end 106.9848 94.7112) (width 0.8) (layer F.Cu) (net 13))
 (segment (start 110.9358 94.742) (end 107.0156 94.742) (width 0.8) (layer F.Cu) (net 13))
 (segment (start 132.7518 101.7524) (end 129.4892 101.7524) (width 0.8) (layer F.Cu) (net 12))
 (segment (start 134.0612 100.443) (end 132.7518 101.7524) (width 0.8) (layer F.Cu) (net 12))
 (segment (start 134.0612 95.3008) (end 134.6708 94.6912) (width 0.8) (layer F.Cu) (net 11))
 (segment (start 134.0612 98.693) (end 134.0612 95.3008) (width 0.8) (layer F.Cu) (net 11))
 (segment (start 137.2108 96.4912) (end 137.2108 94.6912) (width 0.8) (layer F.Cu) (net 4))
 (segment (start 137.2108 96.623702) (end 137.2108 96.4912) (width 0.8) (layer F.Cu) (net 4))
 (segment (start 135.89 97.944502) (end 137.2108 96.623702) (width 0.8) (layer F.Cu) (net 4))
 (segment (start 135.89 103.2764) (end 135.89 97.944502) (width 0.8) (layer F.Cu) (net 4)))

